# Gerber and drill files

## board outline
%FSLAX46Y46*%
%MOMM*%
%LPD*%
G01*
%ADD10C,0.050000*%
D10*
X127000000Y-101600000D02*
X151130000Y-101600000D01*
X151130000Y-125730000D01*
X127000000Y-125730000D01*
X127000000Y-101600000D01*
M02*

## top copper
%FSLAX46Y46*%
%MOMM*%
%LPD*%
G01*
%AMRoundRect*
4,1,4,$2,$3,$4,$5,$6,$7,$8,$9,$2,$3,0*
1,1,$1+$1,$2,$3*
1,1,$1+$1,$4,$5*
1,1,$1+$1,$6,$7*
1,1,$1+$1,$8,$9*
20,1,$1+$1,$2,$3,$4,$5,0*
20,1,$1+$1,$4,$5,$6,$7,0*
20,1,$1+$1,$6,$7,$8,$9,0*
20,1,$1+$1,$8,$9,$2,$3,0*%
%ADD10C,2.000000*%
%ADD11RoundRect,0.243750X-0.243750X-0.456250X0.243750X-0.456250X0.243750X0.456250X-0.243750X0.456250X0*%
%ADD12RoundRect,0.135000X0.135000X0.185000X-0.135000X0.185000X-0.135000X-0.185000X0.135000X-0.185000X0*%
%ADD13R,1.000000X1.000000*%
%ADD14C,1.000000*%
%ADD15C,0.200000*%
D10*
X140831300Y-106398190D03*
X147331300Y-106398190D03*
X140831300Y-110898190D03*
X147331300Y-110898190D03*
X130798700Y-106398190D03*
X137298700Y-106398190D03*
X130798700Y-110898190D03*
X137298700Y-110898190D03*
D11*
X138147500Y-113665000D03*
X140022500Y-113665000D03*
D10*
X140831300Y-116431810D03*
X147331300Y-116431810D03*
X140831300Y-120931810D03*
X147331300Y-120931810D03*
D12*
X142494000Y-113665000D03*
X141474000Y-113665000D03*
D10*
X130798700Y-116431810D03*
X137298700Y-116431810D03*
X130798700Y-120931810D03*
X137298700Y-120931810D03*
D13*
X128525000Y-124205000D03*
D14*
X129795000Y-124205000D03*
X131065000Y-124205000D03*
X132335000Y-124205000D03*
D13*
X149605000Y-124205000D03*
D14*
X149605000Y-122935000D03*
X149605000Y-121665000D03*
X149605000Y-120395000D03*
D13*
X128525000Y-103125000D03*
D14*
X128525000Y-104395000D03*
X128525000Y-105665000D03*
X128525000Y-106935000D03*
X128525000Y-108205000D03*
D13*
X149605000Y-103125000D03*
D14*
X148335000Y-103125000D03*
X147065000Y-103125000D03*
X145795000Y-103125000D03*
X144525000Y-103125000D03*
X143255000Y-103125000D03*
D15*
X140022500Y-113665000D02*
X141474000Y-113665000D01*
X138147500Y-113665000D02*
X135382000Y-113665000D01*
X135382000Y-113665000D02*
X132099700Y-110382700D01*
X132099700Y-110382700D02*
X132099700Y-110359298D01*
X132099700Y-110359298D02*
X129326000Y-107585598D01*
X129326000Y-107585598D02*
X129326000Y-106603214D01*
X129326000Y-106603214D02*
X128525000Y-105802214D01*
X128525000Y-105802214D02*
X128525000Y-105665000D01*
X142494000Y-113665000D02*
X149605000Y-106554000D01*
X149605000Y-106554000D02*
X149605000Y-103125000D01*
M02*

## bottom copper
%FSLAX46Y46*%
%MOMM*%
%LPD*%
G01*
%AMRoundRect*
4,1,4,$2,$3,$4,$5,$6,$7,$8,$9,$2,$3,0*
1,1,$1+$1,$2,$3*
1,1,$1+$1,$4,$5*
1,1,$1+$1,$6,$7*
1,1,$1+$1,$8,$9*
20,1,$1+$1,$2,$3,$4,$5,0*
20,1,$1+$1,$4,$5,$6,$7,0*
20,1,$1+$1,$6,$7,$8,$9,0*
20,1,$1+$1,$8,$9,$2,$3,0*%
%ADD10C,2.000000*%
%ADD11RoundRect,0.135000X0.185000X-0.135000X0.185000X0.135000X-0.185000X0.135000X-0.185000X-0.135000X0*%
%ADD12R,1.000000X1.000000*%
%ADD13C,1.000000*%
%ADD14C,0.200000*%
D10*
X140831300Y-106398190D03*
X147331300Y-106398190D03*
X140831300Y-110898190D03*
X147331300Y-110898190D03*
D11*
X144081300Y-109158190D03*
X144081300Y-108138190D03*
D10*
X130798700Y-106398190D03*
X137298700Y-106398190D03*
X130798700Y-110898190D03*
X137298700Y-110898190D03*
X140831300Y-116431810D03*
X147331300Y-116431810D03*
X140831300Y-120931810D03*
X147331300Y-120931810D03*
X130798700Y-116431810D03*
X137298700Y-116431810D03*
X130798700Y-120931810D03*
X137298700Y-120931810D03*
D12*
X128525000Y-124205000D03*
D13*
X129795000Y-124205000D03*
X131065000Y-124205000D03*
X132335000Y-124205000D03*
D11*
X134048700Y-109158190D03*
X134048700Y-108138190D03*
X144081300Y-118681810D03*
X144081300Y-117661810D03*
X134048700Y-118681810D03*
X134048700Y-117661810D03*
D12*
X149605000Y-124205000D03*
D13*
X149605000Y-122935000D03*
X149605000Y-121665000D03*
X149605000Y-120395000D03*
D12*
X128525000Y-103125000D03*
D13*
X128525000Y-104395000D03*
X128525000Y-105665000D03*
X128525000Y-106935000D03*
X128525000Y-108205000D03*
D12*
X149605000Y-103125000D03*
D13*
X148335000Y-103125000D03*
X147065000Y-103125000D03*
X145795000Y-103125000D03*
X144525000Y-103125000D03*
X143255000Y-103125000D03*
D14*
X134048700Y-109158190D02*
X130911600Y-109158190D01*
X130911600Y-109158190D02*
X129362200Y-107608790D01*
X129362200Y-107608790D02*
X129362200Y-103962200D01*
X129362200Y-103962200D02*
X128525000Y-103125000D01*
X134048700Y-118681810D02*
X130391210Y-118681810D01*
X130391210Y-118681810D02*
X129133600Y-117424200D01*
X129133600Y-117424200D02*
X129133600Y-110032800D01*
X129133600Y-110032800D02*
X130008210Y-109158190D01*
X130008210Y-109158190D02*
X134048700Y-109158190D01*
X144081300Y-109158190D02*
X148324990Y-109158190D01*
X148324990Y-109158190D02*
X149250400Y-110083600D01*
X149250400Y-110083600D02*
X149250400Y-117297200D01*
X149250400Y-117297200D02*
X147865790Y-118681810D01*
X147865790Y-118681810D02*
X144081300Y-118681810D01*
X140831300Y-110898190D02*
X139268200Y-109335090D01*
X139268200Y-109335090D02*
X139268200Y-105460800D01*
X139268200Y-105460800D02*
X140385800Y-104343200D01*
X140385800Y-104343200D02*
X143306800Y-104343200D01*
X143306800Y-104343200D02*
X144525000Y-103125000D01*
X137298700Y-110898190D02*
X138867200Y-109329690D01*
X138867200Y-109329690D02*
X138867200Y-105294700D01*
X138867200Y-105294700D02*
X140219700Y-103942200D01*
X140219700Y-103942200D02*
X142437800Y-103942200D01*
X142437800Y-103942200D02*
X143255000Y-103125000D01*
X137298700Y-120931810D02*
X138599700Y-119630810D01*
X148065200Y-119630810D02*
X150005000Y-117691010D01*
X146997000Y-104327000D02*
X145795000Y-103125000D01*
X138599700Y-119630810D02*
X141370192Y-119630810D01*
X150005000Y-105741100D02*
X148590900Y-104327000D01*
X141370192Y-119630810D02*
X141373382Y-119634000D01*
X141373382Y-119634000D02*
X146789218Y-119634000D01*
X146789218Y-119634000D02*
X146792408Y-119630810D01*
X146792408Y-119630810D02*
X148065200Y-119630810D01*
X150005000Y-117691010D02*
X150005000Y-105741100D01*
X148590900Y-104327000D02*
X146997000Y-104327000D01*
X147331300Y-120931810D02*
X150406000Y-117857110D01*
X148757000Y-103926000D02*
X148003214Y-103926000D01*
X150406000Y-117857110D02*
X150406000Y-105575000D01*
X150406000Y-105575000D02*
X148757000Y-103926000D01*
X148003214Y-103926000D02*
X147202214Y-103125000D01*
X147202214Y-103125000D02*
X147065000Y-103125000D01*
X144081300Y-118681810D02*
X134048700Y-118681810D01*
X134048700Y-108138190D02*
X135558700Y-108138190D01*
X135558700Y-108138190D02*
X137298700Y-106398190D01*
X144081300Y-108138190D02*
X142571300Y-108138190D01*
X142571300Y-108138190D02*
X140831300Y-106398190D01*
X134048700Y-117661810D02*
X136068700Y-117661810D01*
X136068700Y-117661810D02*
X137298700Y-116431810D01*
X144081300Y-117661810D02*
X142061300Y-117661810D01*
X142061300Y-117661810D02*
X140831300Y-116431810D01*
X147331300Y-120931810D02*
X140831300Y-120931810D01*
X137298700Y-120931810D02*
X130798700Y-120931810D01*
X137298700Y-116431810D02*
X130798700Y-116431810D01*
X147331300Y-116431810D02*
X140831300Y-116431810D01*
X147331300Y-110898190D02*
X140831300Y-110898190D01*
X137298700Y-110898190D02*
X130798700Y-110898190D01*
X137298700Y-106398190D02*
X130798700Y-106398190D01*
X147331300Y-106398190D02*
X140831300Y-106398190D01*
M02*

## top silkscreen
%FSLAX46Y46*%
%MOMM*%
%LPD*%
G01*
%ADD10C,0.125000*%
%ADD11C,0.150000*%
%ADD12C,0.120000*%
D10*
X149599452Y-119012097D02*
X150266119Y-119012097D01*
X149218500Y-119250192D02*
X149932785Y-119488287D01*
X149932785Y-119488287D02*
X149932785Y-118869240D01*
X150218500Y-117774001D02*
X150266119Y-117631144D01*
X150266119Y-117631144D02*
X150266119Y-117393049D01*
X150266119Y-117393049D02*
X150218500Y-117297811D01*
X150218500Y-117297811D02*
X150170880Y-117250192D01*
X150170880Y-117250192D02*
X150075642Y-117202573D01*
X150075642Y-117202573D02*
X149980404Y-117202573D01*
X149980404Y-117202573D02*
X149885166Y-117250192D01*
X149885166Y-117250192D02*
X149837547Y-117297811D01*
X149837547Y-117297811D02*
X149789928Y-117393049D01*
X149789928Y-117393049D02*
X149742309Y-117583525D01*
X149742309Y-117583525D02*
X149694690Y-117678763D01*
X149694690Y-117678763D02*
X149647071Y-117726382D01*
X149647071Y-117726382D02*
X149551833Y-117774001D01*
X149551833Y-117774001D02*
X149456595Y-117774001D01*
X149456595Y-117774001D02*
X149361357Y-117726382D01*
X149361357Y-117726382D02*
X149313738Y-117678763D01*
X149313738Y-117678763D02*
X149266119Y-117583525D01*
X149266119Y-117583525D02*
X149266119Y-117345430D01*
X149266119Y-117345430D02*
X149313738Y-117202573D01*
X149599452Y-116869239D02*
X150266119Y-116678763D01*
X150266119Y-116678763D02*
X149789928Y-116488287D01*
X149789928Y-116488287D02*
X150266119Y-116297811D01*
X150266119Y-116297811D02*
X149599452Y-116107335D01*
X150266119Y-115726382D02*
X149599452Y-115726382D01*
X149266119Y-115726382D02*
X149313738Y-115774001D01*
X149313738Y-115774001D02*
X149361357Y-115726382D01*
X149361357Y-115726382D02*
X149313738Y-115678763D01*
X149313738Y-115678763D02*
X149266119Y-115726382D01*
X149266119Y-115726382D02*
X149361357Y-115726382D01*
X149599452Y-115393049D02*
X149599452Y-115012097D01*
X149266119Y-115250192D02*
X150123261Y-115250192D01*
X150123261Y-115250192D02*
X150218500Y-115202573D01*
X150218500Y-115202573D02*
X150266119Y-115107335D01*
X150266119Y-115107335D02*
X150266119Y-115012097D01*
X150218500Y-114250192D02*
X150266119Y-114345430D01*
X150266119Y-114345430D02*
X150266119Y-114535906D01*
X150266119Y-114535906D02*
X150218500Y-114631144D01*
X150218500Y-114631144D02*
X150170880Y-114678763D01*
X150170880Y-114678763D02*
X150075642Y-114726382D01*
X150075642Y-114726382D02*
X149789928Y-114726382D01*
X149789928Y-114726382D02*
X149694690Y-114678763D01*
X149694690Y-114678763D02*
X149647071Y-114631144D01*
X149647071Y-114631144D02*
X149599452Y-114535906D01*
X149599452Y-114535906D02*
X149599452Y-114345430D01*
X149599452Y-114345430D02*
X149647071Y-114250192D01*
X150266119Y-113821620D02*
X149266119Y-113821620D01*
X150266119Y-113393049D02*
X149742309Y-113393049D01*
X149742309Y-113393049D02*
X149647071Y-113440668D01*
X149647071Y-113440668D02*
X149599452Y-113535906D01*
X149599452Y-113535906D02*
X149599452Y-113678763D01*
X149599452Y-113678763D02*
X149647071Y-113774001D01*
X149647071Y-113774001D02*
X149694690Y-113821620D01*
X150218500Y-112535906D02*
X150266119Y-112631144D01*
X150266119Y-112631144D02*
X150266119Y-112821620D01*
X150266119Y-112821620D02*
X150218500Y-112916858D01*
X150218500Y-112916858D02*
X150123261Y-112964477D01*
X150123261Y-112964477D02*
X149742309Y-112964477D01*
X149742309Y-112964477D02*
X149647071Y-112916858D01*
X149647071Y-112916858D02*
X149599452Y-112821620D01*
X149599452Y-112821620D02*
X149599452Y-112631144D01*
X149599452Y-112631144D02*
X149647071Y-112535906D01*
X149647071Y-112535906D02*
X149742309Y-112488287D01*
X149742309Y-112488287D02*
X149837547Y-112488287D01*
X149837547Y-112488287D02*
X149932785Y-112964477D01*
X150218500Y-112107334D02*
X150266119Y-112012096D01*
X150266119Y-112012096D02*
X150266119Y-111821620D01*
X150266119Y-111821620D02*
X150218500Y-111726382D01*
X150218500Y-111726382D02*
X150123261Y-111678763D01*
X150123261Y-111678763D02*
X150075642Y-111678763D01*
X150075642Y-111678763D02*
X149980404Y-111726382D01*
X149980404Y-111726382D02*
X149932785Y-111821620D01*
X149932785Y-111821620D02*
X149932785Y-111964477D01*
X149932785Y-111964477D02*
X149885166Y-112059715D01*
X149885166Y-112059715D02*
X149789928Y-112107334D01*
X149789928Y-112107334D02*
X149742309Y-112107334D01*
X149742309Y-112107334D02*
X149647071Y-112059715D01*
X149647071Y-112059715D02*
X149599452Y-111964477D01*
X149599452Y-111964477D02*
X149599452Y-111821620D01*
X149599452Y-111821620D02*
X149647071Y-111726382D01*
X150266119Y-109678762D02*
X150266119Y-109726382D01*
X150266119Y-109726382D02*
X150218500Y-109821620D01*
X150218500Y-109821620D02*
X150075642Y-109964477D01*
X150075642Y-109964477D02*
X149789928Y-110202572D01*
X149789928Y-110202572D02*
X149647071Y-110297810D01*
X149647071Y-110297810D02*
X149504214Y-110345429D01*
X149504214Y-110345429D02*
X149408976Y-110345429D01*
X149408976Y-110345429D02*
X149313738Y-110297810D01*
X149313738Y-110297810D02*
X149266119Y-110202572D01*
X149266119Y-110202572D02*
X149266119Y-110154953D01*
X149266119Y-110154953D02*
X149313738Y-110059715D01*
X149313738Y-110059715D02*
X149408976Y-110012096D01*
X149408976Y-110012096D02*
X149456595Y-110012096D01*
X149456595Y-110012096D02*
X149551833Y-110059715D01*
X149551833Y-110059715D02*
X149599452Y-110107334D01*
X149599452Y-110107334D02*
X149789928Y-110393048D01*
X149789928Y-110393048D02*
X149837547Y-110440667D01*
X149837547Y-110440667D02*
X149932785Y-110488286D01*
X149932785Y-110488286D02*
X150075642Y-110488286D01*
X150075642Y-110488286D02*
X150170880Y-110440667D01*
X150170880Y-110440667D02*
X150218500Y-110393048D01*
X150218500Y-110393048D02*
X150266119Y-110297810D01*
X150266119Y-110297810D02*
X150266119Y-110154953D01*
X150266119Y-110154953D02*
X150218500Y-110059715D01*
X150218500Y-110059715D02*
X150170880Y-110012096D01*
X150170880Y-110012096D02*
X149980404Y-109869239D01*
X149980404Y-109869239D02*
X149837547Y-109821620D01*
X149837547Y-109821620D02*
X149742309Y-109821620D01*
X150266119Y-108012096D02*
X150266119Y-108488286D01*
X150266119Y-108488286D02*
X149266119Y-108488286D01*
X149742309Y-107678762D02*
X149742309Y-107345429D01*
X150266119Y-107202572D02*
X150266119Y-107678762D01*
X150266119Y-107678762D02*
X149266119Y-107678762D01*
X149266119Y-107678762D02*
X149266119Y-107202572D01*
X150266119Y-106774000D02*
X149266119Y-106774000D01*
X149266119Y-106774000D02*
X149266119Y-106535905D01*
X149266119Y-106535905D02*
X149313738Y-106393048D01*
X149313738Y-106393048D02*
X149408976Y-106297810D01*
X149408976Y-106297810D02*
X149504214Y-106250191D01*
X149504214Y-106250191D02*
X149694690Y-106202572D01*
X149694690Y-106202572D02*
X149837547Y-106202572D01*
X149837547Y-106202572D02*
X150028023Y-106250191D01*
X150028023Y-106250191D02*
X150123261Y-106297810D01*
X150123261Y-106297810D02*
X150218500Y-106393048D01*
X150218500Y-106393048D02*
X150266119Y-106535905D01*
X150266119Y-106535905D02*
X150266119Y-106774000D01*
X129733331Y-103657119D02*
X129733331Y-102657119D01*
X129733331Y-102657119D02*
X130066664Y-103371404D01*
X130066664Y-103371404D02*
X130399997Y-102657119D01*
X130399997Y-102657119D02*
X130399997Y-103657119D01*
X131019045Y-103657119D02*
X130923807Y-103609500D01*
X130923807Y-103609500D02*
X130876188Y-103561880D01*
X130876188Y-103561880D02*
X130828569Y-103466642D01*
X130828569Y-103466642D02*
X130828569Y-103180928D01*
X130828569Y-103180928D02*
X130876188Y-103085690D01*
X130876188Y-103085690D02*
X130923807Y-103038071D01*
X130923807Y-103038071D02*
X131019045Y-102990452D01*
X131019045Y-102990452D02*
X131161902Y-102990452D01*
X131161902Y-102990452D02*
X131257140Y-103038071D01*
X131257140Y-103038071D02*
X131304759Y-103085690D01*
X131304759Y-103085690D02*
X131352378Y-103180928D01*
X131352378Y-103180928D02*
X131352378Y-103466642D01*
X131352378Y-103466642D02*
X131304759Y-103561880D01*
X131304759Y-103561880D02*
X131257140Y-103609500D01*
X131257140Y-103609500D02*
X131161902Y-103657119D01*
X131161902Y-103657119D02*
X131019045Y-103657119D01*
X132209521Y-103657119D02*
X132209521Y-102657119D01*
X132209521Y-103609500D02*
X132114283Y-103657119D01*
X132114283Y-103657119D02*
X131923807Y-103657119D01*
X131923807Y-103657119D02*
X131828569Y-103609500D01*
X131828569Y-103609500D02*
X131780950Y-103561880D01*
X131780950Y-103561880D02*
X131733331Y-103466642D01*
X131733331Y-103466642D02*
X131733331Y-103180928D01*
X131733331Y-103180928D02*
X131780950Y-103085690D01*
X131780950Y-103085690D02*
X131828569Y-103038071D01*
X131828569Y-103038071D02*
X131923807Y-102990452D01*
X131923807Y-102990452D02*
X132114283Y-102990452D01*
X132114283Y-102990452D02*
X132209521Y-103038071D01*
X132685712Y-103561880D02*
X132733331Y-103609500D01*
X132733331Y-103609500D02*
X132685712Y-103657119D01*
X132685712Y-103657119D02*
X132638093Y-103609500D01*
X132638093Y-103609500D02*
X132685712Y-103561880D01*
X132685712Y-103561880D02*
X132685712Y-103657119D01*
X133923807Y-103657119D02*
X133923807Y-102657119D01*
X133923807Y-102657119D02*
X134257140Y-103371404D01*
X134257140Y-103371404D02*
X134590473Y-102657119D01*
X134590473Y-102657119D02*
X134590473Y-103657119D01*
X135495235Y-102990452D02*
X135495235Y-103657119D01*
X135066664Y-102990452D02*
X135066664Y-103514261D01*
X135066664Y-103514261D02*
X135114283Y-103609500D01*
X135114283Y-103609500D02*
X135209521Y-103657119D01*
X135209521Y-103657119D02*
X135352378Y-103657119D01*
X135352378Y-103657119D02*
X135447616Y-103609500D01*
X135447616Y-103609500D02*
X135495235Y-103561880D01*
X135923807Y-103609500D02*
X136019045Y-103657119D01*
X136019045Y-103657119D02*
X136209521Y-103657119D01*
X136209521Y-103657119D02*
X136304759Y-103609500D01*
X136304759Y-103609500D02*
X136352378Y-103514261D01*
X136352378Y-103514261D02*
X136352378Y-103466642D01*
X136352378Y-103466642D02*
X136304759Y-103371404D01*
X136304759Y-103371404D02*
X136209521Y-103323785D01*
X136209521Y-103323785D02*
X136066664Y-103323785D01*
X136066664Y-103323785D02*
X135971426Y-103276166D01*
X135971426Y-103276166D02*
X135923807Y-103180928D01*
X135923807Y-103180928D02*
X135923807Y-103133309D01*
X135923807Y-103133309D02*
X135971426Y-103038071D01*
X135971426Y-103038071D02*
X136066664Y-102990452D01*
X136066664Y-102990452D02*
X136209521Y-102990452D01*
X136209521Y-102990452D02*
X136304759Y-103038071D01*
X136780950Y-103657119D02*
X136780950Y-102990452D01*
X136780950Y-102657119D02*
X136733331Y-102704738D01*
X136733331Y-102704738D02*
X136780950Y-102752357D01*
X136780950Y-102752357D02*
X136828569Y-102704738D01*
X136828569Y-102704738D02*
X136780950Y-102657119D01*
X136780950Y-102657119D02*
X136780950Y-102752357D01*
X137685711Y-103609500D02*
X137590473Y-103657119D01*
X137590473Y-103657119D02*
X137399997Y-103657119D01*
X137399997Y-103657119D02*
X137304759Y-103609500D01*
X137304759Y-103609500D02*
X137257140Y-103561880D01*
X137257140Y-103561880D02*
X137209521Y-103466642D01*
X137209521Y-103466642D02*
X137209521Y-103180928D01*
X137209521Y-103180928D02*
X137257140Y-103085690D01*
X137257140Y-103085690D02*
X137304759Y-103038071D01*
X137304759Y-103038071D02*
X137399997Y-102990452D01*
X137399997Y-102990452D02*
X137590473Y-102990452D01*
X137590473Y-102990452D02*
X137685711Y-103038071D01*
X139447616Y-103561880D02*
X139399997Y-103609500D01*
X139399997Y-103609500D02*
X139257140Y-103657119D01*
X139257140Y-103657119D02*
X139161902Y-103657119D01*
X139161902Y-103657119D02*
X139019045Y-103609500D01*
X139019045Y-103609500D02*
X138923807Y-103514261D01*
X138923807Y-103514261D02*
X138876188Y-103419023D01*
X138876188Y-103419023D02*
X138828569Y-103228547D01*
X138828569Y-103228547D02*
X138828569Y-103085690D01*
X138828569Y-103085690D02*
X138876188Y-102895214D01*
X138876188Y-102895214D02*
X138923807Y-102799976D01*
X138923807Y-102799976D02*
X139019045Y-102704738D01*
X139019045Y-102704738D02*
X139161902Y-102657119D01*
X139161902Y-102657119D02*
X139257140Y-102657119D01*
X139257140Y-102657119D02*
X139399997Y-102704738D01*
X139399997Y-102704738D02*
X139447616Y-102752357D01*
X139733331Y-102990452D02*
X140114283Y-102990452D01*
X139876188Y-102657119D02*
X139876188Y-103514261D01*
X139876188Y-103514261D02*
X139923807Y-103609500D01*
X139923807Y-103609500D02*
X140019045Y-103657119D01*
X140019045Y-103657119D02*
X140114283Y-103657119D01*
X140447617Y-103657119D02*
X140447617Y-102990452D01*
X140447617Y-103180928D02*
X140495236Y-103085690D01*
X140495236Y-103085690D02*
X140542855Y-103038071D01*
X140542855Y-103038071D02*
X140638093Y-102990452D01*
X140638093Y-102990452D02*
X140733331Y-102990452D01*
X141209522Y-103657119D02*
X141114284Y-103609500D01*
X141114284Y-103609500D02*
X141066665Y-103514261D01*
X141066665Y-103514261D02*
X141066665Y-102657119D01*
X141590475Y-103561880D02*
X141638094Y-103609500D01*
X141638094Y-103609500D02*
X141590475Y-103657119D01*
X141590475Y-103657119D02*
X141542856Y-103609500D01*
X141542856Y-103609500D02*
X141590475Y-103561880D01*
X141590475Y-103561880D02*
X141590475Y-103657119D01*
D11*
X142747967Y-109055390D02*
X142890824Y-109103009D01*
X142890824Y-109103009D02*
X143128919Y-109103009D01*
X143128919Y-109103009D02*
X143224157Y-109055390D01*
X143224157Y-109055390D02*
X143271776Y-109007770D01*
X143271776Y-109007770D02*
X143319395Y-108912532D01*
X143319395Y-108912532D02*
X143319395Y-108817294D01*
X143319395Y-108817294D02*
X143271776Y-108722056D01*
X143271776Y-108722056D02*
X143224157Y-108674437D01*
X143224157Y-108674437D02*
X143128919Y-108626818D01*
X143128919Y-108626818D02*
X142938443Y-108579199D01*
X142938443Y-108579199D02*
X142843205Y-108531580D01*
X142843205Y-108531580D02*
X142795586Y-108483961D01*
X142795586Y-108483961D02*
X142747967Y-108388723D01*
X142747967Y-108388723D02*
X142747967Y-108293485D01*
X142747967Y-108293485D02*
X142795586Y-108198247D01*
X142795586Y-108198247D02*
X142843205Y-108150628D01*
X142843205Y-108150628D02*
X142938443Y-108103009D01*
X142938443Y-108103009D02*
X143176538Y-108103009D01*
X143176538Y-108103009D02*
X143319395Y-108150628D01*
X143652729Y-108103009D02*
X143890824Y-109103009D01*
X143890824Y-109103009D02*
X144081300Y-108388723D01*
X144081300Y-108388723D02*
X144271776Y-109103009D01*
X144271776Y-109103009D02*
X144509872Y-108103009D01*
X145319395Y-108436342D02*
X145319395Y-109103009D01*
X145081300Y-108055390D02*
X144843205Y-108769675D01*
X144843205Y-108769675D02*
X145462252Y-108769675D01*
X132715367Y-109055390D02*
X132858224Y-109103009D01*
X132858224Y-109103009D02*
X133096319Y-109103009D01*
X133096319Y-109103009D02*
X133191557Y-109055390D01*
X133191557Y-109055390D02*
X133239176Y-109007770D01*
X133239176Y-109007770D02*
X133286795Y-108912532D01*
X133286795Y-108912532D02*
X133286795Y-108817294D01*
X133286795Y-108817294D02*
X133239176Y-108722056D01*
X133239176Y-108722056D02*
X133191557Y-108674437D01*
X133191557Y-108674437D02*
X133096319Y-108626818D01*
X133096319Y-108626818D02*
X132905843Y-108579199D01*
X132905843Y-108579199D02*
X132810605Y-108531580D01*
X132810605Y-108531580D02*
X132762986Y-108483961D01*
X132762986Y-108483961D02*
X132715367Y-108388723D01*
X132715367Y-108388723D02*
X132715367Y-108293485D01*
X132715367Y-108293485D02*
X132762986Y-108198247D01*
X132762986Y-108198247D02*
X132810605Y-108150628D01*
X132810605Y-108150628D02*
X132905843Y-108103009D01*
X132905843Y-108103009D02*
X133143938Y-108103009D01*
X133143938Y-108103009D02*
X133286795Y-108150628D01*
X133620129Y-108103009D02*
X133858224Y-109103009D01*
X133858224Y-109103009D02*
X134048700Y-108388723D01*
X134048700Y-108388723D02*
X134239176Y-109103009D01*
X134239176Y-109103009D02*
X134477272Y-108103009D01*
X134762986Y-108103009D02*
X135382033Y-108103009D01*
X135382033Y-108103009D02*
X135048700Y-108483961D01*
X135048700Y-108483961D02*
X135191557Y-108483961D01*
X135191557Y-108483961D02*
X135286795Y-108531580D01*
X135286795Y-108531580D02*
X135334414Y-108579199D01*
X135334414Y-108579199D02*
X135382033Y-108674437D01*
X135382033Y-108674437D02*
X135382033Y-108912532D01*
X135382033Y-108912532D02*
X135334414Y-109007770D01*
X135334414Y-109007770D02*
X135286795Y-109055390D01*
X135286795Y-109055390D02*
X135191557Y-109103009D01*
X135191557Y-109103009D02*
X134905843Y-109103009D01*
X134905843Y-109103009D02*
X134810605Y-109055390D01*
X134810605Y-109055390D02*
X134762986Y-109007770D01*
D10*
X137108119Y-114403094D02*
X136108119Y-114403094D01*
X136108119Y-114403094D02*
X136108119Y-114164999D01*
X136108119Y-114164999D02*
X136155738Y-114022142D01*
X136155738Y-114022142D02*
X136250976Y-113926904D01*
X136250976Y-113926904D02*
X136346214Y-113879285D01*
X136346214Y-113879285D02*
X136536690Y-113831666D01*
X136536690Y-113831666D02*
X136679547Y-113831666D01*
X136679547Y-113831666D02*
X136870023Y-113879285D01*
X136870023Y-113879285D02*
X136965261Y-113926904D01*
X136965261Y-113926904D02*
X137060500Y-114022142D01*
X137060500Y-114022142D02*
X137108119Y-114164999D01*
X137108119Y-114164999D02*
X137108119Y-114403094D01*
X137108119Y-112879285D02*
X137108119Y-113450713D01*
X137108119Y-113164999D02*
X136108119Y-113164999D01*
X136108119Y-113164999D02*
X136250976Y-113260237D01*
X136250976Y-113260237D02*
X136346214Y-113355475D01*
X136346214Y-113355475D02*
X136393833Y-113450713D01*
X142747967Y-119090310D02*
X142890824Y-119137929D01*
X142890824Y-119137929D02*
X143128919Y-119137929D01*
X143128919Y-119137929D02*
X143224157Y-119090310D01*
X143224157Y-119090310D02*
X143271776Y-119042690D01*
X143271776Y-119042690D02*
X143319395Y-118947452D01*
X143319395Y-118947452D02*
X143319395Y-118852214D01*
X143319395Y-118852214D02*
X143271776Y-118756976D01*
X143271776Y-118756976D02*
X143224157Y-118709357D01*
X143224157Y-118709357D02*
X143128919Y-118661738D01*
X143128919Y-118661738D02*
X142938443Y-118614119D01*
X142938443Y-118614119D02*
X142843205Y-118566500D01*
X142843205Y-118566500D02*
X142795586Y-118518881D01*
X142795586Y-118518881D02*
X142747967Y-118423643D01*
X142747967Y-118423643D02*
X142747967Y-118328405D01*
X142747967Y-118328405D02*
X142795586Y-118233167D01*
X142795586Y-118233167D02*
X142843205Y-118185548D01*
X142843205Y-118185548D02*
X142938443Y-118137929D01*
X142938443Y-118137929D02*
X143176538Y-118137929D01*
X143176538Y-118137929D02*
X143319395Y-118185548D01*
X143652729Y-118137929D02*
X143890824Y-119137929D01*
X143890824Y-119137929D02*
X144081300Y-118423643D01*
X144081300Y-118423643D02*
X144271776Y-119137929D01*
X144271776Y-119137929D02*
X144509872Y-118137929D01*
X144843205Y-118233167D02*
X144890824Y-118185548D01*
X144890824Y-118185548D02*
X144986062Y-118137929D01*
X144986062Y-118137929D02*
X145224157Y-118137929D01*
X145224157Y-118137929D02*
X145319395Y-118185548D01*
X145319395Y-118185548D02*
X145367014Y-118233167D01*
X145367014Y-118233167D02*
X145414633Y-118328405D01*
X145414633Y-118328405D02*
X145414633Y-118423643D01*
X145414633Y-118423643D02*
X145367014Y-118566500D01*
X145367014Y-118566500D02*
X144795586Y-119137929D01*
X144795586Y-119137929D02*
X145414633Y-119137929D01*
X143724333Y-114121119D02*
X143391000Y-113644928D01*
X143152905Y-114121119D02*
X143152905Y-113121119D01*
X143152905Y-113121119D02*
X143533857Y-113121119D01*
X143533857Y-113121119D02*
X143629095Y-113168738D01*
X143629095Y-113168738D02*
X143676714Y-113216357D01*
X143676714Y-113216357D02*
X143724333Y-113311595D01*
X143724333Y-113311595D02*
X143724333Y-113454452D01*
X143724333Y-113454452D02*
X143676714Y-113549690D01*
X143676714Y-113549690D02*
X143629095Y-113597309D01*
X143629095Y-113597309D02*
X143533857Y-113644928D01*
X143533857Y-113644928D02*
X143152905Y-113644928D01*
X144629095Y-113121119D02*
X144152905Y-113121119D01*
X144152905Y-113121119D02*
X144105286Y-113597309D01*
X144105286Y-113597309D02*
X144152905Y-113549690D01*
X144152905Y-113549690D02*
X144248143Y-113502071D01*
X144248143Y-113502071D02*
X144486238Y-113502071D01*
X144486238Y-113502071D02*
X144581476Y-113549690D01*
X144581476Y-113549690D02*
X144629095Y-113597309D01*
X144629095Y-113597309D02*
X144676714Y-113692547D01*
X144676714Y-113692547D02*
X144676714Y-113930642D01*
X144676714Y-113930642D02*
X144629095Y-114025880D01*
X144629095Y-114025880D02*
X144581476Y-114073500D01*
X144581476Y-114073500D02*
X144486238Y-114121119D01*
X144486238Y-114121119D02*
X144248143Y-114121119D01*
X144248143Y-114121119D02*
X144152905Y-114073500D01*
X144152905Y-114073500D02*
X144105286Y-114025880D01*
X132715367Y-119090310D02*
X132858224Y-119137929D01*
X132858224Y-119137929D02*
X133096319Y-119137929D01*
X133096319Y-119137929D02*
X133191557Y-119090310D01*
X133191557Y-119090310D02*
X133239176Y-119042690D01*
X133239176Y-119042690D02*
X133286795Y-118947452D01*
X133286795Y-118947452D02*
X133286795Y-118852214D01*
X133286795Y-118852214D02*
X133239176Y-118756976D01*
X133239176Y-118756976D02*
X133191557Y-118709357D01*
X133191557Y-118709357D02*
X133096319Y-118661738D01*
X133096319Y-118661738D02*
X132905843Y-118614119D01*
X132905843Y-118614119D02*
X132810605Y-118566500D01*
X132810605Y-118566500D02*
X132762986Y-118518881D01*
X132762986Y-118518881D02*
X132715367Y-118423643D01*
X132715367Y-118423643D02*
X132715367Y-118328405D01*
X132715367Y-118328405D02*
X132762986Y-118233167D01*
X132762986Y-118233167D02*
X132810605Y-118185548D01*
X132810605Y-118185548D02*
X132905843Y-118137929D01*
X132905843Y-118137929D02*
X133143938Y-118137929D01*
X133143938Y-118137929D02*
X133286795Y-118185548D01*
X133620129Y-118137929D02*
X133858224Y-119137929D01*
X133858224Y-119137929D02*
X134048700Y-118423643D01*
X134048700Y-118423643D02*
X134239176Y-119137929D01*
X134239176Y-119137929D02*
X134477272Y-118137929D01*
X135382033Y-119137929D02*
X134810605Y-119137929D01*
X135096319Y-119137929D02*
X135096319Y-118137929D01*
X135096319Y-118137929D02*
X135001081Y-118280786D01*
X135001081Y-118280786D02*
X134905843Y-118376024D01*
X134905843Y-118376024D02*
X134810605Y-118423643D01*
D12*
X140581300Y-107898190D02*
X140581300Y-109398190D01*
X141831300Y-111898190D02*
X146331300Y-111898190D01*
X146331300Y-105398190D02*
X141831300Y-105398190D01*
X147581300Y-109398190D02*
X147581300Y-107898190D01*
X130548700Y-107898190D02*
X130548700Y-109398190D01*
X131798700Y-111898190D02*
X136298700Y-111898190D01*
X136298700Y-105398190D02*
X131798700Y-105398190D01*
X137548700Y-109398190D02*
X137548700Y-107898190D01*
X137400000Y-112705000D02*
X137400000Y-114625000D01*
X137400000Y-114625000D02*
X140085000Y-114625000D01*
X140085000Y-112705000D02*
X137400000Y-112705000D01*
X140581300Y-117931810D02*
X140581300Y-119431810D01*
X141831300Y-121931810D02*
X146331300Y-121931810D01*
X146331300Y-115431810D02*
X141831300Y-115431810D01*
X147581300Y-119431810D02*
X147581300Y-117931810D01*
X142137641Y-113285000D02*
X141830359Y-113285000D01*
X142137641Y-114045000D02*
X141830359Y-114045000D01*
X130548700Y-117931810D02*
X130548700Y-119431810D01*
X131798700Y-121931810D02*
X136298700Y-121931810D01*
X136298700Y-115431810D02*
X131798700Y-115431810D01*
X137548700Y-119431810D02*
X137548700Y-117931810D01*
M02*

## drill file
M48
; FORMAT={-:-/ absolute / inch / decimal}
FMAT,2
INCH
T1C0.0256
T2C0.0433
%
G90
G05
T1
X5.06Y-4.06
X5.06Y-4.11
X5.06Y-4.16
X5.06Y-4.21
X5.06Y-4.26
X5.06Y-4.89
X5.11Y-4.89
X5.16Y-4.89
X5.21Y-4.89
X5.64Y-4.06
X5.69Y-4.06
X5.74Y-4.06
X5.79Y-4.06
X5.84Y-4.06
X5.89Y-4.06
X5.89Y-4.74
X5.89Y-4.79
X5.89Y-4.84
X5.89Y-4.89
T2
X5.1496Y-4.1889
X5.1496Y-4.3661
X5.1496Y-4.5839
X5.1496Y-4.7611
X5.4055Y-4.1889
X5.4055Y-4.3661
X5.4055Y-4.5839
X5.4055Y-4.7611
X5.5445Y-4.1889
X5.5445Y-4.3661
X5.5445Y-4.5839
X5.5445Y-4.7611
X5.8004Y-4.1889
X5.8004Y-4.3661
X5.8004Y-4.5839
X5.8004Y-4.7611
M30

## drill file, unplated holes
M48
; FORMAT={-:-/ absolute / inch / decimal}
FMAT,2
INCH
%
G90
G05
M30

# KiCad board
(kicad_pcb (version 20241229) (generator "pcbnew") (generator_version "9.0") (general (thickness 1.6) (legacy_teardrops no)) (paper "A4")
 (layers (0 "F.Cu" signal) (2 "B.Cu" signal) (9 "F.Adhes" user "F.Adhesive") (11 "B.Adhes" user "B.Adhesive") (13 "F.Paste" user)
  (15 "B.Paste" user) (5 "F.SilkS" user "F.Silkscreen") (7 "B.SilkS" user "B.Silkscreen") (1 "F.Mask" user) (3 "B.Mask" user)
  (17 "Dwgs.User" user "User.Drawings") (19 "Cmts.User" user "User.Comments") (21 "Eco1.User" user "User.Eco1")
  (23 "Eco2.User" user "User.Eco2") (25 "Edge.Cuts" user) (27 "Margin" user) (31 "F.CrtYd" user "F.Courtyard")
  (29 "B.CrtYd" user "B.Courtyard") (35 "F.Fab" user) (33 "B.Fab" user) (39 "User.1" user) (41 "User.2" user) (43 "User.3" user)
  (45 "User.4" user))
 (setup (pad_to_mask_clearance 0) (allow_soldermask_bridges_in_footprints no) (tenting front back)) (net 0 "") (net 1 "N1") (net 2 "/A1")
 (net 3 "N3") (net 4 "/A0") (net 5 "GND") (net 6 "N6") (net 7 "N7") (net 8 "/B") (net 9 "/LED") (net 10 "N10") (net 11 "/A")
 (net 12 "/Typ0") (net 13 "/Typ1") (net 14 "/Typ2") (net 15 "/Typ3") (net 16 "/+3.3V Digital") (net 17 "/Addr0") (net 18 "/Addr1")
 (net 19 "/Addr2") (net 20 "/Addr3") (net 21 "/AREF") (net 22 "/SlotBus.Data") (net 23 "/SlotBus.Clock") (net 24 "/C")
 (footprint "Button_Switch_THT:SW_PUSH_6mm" (layer "F.Cu") (at 140.8313 106.39819)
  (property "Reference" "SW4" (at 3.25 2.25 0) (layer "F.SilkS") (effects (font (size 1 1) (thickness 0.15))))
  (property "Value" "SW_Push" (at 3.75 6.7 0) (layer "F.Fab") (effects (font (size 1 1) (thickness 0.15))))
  (fp_line (start -0.25 1.5) (end -0.25 3) (stroke (width 0.12) (type solid)) (layer "F.SilkS"))
  (fp_line (start 1 5.5) (end 5.5 5.5) (stroke (width 0.12) (type solid)) (layer "F.SilkS"))
  (fp_line (start 5.5 -1) (end 1 -1) (stroke (width 0.12) (type solid)) (layer "F.SilkS"))
  (fp_line (start 6.75 3) (end 6.75 1.5) (stroke (width 0.12) (type solid)) (layer "F.SilkS"))
  (pad "1" thru_hole circle (at 0 0 90) (size 2 2) (drill 1.1) (layers "*.Cu" "*.Mask") (remove_unused_layers no) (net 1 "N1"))
  (pad "1" thru_hole circle (at 6.5 0 90) (size 2 2) (drill 1.1) (layers "*.Cu" "*.Mask") (remove_unused_layers no) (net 1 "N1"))
  (pad "2" thru_hole circle (at 0 4.5 90) (size 2 2) (drill 1.1) (layers "*.Cu" "*.Mask") (remove_unused_layers no) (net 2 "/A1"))
  (pad "2" thru_hole circle (at 6.5 4.5 90) (size 2 2) (drill 1.1) (layers "*.Cu" "*.Mask") (remove_unused_layers no) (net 2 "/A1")))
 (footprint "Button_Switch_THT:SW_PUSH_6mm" (layer "F.Cu") (at 130.7987 106.39819)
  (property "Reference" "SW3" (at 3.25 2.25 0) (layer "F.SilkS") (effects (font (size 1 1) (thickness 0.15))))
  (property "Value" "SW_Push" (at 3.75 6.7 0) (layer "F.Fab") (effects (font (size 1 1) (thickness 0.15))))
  (fp_line (start -0.25 1.5) (end -0.25 3) (stroke (width 0.12) (type solid)) (layer "F.SilkS"))
  (fp_line (start 1 5.5) (end 5.5 5.5) (stroke (width 0.12) (type solid)) (layer "F.SilkS"))
  (fp_line (start 5.5 -1) (end 1 -1) (stroke (width 0.12) (type solid)) (layer "F.SilkS"))
  (fp_line (start 6.75 3) (end 6.75 1.5) (stroke (width 0.12) (type solid)) (layer "F.SilkS"))
  (pad "1" thru_hole circle (at 0 0 90) (size 2 2) (drill 1.1) (layers "*.Cu" "*.Mask") (remove_unused_layers no) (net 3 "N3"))
  (pad "1" thru_hole circle (at 6.5 0 90) (size 2 2) (drill 1.1) (layers "*.Cu" "*.Mask") (remove_unused_layers no) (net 3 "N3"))
  (pad "2" thru_hole circle (at 0 4.5 90) (size 2 2) (drill 1.1) (layers "*.Cu" "*.Mask") (remove_unused_layers no) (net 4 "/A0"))
  (pad "2" thru_hole circle (at 6.5 4.5 90) (size 2 2) (drill 1.1) (layers "*.Cu" "*.Mask") (remove_unused_layers no) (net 4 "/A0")))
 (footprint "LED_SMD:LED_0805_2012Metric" (layer "F.Cu") (at 139.085 113.665)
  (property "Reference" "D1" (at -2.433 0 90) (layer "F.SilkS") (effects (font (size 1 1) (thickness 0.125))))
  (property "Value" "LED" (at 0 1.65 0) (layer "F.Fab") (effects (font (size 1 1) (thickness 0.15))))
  (fp_line (start -1.685 -0.96) (end -1.685 0.96) (stroke (width 0.12) (type solid)) (layer "F.SilkS"))
  (fp_line (start -1.685 0.96) (end 1 0.96) (stroke (width 0.12) (type solid)) (layer "F.SilkS"))
  (fp_line (start 1 -0.96) (end -1.685 -0.96) (stroke (width 0.12) (type solid)) (layer "F.SilkS"))
  (pad "1" smd roundrect (at -0.9375 0) (size 0.975 1.4) (layers "F.Cu" "F.Mask" "F.Paste") (roundrect_rratio 0.25) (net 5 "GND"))
  (pad "2" smd roundrect (at 0.9375 0) (size 0.975 1.4) (layers "F.Cu" "F.Mask" "F.Paste") (roundrect_rratio 0.25) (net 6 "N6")))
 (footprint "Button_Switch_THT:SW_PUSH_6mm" (layer "F.Cu") (at 140.8313 116.43181)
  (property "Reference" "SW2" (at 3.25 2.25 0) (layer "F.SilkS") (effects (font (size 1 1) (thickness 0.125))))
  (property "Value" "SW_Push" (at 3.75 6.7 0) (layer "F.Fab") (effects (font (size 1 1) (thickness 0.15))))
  (fp_line (start -0.25 1.5) (end -0.25 3) (stroke (width 0.12) (type solid)) (layer "F.SilkS"))
  (fp_line (start 1 5.5) (end 5.5 5.5) (stroke (width 0.12) (type solid)) (layer "F.SilkS"))
  (fp_line (start 5.5 -1) (end 1 -1) (stroke (width 0.12) (type solid)) (layer "F.SilkS"))
  (fp_line (start 6.75 3) (end 6.75 1.5) (stroke (width 0.12) (type solid)) (layer "F.SilkS"))
  (pad "1" thru_hole circle (at 0 0 90) (size 2 2) (drill 1.1) (layers "*.Cu" "*.Mask") (remove_unused_layers no) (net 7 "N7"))
  (pad "1" thru_hole circle (at 6.5 0 90) (size 2 2) (drill 1.1) (layers "*.Cu" "*.Mask") (remove_unused_layers no) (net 7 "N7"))
  (pad "2" thru_hole circle (at 0 4.5 90) (size 2 2) (drill 1.1) (layers "*.Cu" "*.Mask") (remove_unused_layers no) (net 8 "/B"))
  (pad "2" thru_hole circle (at 6.5 4.5 90) (size 2 2) (drill 1.1) (layers "*.Cu" "*.Mask") (remove_unused_layers no) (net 8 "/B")))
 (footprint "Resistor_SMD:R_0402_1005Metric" (layer "F.Cu") (at 141.984 113.665 180)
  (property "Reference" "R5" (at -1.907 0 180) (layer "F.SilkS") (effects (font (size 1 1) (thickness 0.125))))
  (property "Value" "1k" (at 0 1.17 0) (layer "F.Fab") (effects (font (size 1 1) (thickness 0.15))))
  (fp_line (start -0.153641 0.38) (end 0.153641 0.38) (stroke (width 0.12) (type solid)) (layer "F.SilkS"))
  (fp_line (start -0.153641 -0.38) (end 0.153641 -0.38) (stroke (width 0.12) (type solid)) (layer "F.SilkS"))
  (pad "1" smd roundrect (at -0.51 0 180) (size 0.54 0.64) (layers "F.Cu" "F.Mask" "F.Paste") (roundrect_rratio 0.25) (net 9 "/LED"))
  (pad "2" smd roundrect (at 0.51 0 180) (size 0.54 0.64) (layers "F.Cu" "F.Mask" "F.Paste") (roundrect_rratio 0.25) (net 6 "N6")))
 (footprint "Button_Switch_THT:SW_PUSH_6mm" (layer "F.Cu") (at 130.7987 116.43181)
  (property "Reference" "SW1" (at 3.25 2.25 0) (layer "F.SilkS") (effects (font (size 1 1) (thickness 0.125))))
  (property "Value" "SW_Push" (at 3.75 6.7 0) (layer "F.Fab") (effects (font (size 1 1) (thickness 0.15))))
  (fp_line (start -0.25 1.5) (end -0.25 3) (stroke (width 0.12) (type solid)) (layer "F.SilkS"))
  (fp_line (start 1 5.5) (end 5.5 5.5) (stroke (width 0.12) (type solid)) (layer "F.SilkS"))
  (fp_line (start 5.5 -1) (end 1 -1) (stroke (width 0.12) (type solid)) (layer "F.SilkS"))
  (fp_line (start 6.75 3) (end 6.75 1.5) (stroke (width 0.12) (type solid)) (layer "F.SilkS"))
  (pad "1" thru_hole circle (at 0 0 90) (size 2 2) (drill 1.1) (layers "*.Cu" "*.Mask") (remove_unused_layers no) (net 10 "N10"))
  (pad "1" thru_hole circle (at 6.5 0 90) (size 2 2) (drill 1.1) (layers "*.Cu" "*.Mask") (remove_unused_layers no) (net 10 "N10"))
  (pad "2" thru_hole circle (at 0 4.5 90) (size 2 2) (drill 1.1) (layers "*.Cu" "*.Mask") (remove_unused_layers no) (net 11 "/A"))
  (pad "2" thru_hole circle (at 6.5 4.5 90) (size 2 2) (drill 1.1) (layers "*.Cu" "*.Mask") (remove_unused_layers no) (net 11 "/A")))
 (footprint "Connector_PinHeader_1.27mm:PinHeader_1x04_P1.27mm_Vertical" (layer "B.Cu") (at 128.525 124.205 -90)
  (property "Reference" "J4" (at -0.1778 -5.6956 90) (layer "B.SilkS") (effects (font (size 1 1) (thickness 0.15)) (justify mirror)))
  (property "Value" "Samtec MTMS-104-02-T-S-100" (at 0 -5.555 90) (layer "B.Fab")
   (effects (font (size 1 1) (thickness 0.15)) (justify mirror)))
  (pad "1" thru_hole rect (at 0 0 270) (size 1 1) (drill 0.65) (layers "*.Cu" "*.Mask") (remove_unused_layers no) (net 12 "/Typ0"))
  (pad "2" thru_hole circle (at 0 -1.27 270) (size 1 1) (drill 0.65) (layers "*.Cu" "*.Mask") (remove_unused_layers no) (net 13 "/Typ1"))
  (pad "3" thru_hole circle (at 0 -2.54 270) (size 1 1) (drill 0.65) (layers "*.Cu" "*.Mask") (remove_unused_layers no) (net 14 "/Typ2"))
  (pad "4" thru_hole circle (at 0 -3.81 270) (size 1 1) (drill 0.65) (layers "*.Cu" "*.Mask") (remove_unused_layers no) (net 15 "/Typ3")))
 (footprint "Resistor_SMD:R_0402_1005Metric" (layer "B.Cu") (at 134.0487 108.64819 90)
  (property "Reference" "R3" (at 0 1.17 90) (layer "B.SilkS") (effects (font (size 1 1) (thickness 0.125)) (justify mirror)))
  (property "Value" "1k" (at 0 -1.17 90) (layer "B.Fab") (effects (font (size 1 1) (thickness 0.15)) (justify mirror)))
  (pad "1" smd roundrect (at -0.51 0 90) (size 0.54 0.64) (layers "B.Cu" "B.Mask" "B.Paste") (roundrect_rratio 0.25)
   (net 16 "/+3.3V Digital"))
  (pad "2" smd roundrect (at 0.51 0 90) (size 0.54 0.64) (layers "B.Cu" "B.Mask" "B.Paste") (roundrect_rratio 0.25) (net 3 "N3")))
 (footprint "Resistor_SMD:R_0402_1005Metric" (layer "B.Cu") (at 144.0813 118.17181 90)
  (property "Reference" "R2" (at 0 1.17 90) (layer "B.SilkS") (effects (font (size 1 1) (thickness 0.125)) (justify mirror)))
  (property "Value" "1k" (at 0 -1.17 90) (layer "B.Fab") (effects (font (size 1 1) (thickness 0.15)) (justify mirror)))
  (pad "1" smd roundrect (at -0.51 0 90) (size 0.54 0.64) (layers "B.Cu" "B.Mask" "B.Paste") (roundrect_rratio 0.25)
   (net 16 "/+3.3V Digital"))
  (pad "2" smd roundrect (at 0.51 0 90) (size 0.54 0.64) (layers "B.Cu" "B.Mask" "B.Paste") (roundrect_rratio 0.25) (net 7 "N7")))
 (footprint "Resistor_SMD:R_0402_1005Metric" (layer "B.Cu") (at 134.0487 118.17181 90)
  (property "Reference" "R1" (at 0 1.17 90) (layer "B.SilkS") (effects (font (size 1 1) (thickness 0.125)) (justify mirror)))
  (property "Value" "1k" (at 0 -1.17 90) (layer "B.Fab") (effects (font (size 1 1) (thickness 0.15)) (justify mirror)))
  (pad "1" smd roundrect (at -0.51 0 90) (size 0.54 0.64) (layers "B.Cu" "B.Mask" "B.Paste") (roundrect_rratio 0.25)
   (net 16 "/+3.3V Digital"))
  (pad "2" smd roundrect (at 0.51 0 90) (size 0.54 0.64) (layers "B.Cu" "B.Mask" "B.Paste") (roundrect_rratio 0.25) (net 10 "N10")))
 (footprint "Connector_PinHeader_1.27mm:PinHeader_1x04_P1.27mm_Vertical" (layer "B.Cu") (at 149.605 124.205)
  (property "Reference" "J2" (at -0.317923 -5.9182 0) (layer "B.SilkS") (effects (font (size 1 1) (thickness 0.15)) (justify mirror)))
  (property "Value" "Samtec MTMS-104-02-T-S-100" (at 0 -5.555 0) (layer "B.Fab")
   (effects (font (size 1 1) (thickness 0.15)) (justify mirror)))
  (pad "1" thru_hole rect (at 0 0) (size 1 1) (drill 0.65) (layers "*.Cu" "*.Mask") (remove_unused_layers no) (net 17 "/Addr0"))
  (pad "2" thru_hole circle (at 0 -1.27) (size 1 1) (drill 0.65) (layers "*.Cu" "*.Mask") (remove_unused_layers no) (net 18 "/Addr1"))
  (pad "3" thru_hole circle (at 0 -2.54) (size 1 1) (drill 0.65) (layers "*.Cu" "*.Mask") (remove_unused_layers no) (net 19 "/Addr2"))
  (pad "4" thru_hole circle (at 0 -3.81) (size 1 1) (drill 0.65) (layers "*.Cu" "*.Mask") (remove_unused_layers no) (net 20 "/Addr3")))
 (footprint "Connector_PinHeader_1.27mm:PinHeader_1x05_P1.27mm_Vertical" (layer "B.Cu") (at 128.525 103.125 180)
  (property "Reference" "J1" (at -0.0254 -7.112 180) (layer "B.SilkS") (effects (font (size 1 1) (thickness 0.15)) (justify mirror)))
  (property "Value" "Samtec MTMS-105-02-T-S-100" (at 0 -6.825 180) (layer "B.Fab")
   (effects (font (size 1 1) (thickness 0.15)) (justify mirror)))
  (pad "1" thru_hole rect (at 0 0 180) (size 1 1) (drill 0.65) (layers "*.Cu" "*.Mask") (remove_unused_layers no) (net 16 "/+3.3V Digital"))
  (pad "2" thru_hole circle (at 0 -1.27 180) (size 1 1) (drill 0.65) (layers "*.Cu" "*.Mask") (remove_unused_layers no) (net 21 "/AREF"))
  (pad "3" thru_hole circle (at 0 -2.54 180) (size 1 1) (drill 0.65) (layers "*.Cu" "*.Mask") (remove_unused_layers no) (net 5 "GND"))
  (pad "4" thru_hole circle (at 0 -3.81 180) (size 1 1) (drill 0.65) (layers "*.Cu" "*.Mask") (remove_unused_layers no)
   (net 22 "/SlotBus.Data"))
  (pad "5" thru_hole circle (at 0 -5.08 180) (size 1 1) (drill 0.65) (layers "*.Cu" "*.Mask") (remove_unused_layers no)
   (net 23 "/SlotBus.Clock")))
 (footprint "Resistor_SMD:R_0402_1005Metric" (layer "B.Cu") (at 144.0813 108.64819 90)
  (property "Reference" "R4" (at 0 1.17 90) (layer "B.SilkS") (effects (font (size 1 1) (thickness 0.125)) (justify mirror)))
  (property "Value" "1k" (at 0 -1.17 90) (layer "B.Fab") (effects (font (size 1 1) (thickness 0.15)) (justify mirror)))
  (pad "1" smd roundrect (at -0.51 0 90) (size 0.54 0.64) (layers "B.Cu" "B.Mask" "B.Paste") (roundrect_rratio 0.25)
   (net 16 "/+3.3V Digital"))
  (pad "2" smd roundrect (at 0.51 0 90) (size 0.54 0.64) (layers "B.Cu" "B.Mask" "B.Paste") (roundrect_rratio 0.25) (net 1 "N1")))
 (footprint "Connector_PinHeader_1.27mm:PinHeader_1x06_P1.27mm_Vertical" (layer "B.Cu") (at 149.605 103.125 90)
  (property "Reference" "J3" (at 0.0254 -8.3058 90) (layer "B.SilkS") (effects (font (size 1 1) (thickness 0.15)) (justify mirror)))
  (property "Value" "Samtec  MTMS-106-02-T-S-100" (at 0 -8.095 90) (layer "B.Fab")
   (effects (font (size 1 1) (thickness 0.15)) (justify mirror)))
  (pad "1" thru_hole rect (at 0 0 90) (size 1 1) (drill 0.65) (layers "*.Cu" "*.Mask") (remove_unused_layers no) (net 9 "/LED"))
  (pad "2" thru_hole circle (at 0 -1.27 90) (size 1 1) (drill 0.65) (layers "*.Cu" "*.Mask") (remove_unused_layers no) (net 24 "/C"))
  (pad "3" thru_hole circle (at 0 -2.54 90) (size 1 1) (drill 0.65) (layers "*.Cu" "*.Mask") (remove_unused_layers no) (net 8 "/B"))
  (pad "4" thru_hole circle (at 0 -3.81 90) (size 1 1) (drill 0.65) (layers "*.Cu" "*.Mask") (remove_unused_layers no) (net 11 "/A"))
  (pad "5" thru_hole circle (at 0 -5.08 90) (size 1 1) (drill 0.65) (layers "*.Cu" "*.Mask") (remove_unused_layers no) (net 2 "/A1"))
  (pad "6" thru_hole circle (at 0 -6.35 90) (size 1 1) (drill 0.65) (layers "*.Cu" "*.Mask") (remove_unused_layers no) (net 4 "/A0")))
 (gr_rect (start 127 101.6) (end 151.13 125.73) (stroke (width 0.05) (type solid)) (fill no) (layer "Edge.Cuts"))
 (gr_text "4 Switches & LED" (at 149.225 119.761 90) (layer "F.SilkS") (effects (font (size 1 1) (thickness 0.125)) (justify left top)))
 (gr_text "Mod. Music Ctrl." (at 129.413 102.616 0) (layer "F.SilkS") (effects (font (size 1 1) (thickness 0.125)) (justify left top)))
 (segment (start 138.1475 113.665) (end 135.382 113.665) (width 0.2) (layer "F.Cu") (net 5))
 (segment (start 129.326 107.585598) (end 129.326 106.603214) (width 0.2) (layer "F.Cu") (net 5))
 (segment (start 129.326 106.603214) (end 128.525 105.802214) (width 0.2) (layer "F.Cu") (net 5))
 (segment (start 132.0997 110.3827) (end 132.0997 110.359298) (width 0.2) (layer "F.Cu") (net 5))
 (segment (start 128.525 105.802214) (end 128.525 105.665) (width 0.2) (layer "F.Cu") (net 5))
 (segment (start 132.0997 110.359298) (end 129.326 107.585598) (width 0.2) (layer "F.Cu") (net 5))
 (segment (start 135.382 113.665) (end 132.0997 110.3827) (width 0.2) (layer "F.Cu") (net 5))
 (segment (start 140.0225 113.665) (end 141.474 113.665) (width 0.2) (layer "F.Cu") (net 6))
 (segment (start 129.1336 110.0328) (end 130.00821 109.15819) (width 0.2) (layer "B.Cu") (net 16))
 (segment (start 129.1336 117.4242) (end 129.1336 110.0328) (width 0.2) (layer "B.Cu") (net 16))
 (segment (start 148.32499 109.15819) (end 149.2504 110.0836) (width 0.2) (layer "B.Cu") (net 16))
 (segment (start 144.0813 118.68181) (end 134.0487 118.68181) (width 0.2) (layer "B.Cu") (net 16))
 (segment (start 149.2504 117.2972) (end 147.86579 118.68181) (width 0.2) (layer "B.Cu") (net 16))
 (segment (start 134.0487 118.68181) (end 130.39121 118.68181) (width 0.2) (layer "B.Cu") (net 16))
 (segment (start 129.3622 103.9622) (end 128.525 103.125) (width 0.2) (layer "B.Cu") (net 16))
 (segment (start 130.39121 118.68181) (end 129.1336 117.4242) (width 0.2) (layer "B.Cu") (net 16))
 (segment (start 149.2504 110.0836) (end 149.2504 117.2972) (width 0.2) (layer "B.Cu") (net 16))
 (segment (start 144.0813 109.15819) (end 148.32499 109.15819) (width 0.2) (layer "B.Cu") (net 16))
 (segment (start 130.9116 109.15819) (end 129.3622 107.60879) (width 0.2) (layer "B.Cu") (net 16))
 (segment (start 134.0487 109.15819) (end 130.9116 109.15819) (width 0.2) (layer "B.Cu") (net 16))
 (segment (start 147.86579 118.68181) (end 144.0813 118.68181) (width 0.2) (layer "B.Cu") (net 16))
 (segment (start 129.3622 107.60879) (end 129.3622 103.9622) (width 0.2) (layer "B.Cu") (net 16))
 (segment (start 130.00821 109.15819) (end 134.0487 109.15819) (width 0.2) (layer "B.Cu") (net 16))
 (segment (start 148.757 103.926) (end 148.003214 103.926) (width 0.2) (layer "B.Cu") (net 8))
 (segment (start 150.406 105.575) (end 148.757 103.926) (width 0.2) (layer "B.Cu") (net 8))
 (segment (start 150.406 117.85711) (end 150.406 105.575) (width 0.2) (layer "B.Cu") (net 8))
 (segment (start 148.003214 103.926) (end 147.202214 103.125) (width 0.2) (layer "B.Cu") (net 8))
 (segment (start 147.202214 103.125) (end 147.065 103.125) (width 0.2) (layer "B.Cu") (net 8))
 (segment (start 147.3313 120.93181) (end 140.8313 120.93181) (width 0.2) (layer "B.Cu") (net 8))
 (segment (start 147.3313 120.93181) (end 150.406 117.85711) (width 0.2) (layer "B.Cu") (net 8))
 (segment (start 142.494 113.665) (end 149.605 106.554) (width 0.2) (layer "F.Cu") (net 9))
 (segment (start 149.605 106.554) (end 149.605 103.125) (width 0.2) (layer "F.Cu") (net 9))
 (segment (start 147.3313 110.89819) (end 140.8313 110.89819) (width 0.2) (layer "B.Cu") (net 2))
 (segment (start 139.2682 105.4608) (end 140.3858 104.3432) (width 0.2) (layer "B.Cu") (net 2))
 (segment (start 140.8313 110.89819) (end 139.2682 109.33509) (width 0.2) (layer "B.Cu") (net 2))
 (segment (start 140.3858 104.3432) (end 143.3068 104.3432) (width 0.2) (layer "B.Cu") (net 2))
 (segment (start 143.3068 104.3432) (end 144.525 103.125) (width 0.2) (layer "B.Cu") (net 2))
 (segment (start 139.2682 109.33509) (end 139.2682 105.4608) (width 0.2) (layer "B.Cu") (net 2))
 (segment (start 137.2987 120.93181) (end 130.7987 120.93181) (width 0.2) (layer "B.Cu") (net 11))
 (segment (start 141.373382 119.634) (end 146.789218 119.634) (width 0.2) (layer "B.Cu") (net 11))
 (segment (start 148.5909 104.327) (end 146.997 104.327) (width 0.2) (layer "B.Cu") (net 11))
 (segment (start 141.370192 119.63081) (end 141.373382 119.634) (width 0.2) (layer "B.Cu") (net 11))
 (segment (start 150.005 105.7411) (end 148.5909 104.327) (width 0.2) (layer "B.Cu") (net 11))
 (segment (start 137.2987 120.93181) (end 138.5997 119.63081) (width 0.2) (layer "B.Cu") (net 11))
 (segment (start 148.0652 119.63081) (end 150.005 117.69101) (width 0.2) (layer "B.Cu") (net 11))
 (segment (start 146.792408 119.63081) (end 148.0652 119.63081) (width 0.2) (layer "B.Cu") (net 11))
 (segment (start 146.789218 119.634) (end 146.792408 119.63081) (width 0.2) (layer "B.Cu") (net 11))
 (segment (start 146.997 104.327) (end 145.795 103.125) (width 0.2) (layer "B.Cu") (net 11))
 (segment (start 150.005 117.69101) (end 150.005 105.7411) (width 0.2) (layer "B.Cu") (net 11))
 (segment (start 138.5997 119.63081) (end 141.370192 119.63081) (width 0.2) (layer "B.Cu") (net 11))
 (segment (start 140.2197 103.9422) (end 142.4378 103.9422) (width 0.2) (layer "B.Cu") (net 4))
 (segment (start 142.4378 103.9422) (end 143.255 103.125) (width 0.2) (layer "B.Cu") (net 4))
 (segment (start 138.8672 109.32969) (end 138.8672 105.2947) (width 0.2) (layer "B.Cu") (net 4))
 (segment (start 138.8672 105.2947) (end 140.2197 103.9422) (width 0.2) (layer "B.Cu") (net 4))
 (segment (start 137.2987 110.89819) (end 130.7987 110.89819) (width 0.2) (layer "B.Cu") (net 4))
 (segment (start 137.2987 110.89819) (end 138.8672 109.32969) (width 0.2) (layer "B.Cu") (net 4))
 (segment (start 134.0487 117.66181) (end 136.0687 117.66181) (width 0.2) (layer "B.Cu") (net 10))
 (segment (start 136.0687 117.66181) (end 137.2987 116.43181) (width 0.2) (layer "B.Cu") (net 10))
 (segment (start 137.2987 116.43181) (end 130.7987 116.43181) (width 0.2) (layer "B.Cu") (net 10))
 (segment (start 144.0813 117.66181) (end 142.0613 117.66181) (width 0.2) (layer "B.Cu") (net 7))
 (segment (start 142.0613 117.66181) (end 140.8313 116.43181) (width 0.2) (layer "B.Cu") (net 7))
 (segment (start 147.3313 116.43181) (end 140.8313 116.43181) (width 0.2) (layer "B.Cu") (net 7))
 (segment (start 134.0487 108.13819) (end 135.5587 108.13819) (width 0.2) (layer "B.Cu") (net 3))
 (segment (start 135.5587 108.13819) (end 137.2987 106.39819) (width 0.2) (layer "B.Cu") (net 3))
 (segment (start 137.2987 106.39819) (end 130.7987 106.39819) (width 0.2) (layer "B.Cu") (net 3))
 (segment (start 142.5713 108.13819) (end 140.8313 106.39819) (width 0.2) (layer "B.Cu") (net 1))
 (segment (start 147.3313 106.39819) (end 140.8313 106.39819) (width 0.2) (layer "B.Cu") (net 1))
 (segment (start 144.0813 108.13819) (end 142.5713 108.13819) (width 0.2) (layer "B.Cu") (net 1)))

